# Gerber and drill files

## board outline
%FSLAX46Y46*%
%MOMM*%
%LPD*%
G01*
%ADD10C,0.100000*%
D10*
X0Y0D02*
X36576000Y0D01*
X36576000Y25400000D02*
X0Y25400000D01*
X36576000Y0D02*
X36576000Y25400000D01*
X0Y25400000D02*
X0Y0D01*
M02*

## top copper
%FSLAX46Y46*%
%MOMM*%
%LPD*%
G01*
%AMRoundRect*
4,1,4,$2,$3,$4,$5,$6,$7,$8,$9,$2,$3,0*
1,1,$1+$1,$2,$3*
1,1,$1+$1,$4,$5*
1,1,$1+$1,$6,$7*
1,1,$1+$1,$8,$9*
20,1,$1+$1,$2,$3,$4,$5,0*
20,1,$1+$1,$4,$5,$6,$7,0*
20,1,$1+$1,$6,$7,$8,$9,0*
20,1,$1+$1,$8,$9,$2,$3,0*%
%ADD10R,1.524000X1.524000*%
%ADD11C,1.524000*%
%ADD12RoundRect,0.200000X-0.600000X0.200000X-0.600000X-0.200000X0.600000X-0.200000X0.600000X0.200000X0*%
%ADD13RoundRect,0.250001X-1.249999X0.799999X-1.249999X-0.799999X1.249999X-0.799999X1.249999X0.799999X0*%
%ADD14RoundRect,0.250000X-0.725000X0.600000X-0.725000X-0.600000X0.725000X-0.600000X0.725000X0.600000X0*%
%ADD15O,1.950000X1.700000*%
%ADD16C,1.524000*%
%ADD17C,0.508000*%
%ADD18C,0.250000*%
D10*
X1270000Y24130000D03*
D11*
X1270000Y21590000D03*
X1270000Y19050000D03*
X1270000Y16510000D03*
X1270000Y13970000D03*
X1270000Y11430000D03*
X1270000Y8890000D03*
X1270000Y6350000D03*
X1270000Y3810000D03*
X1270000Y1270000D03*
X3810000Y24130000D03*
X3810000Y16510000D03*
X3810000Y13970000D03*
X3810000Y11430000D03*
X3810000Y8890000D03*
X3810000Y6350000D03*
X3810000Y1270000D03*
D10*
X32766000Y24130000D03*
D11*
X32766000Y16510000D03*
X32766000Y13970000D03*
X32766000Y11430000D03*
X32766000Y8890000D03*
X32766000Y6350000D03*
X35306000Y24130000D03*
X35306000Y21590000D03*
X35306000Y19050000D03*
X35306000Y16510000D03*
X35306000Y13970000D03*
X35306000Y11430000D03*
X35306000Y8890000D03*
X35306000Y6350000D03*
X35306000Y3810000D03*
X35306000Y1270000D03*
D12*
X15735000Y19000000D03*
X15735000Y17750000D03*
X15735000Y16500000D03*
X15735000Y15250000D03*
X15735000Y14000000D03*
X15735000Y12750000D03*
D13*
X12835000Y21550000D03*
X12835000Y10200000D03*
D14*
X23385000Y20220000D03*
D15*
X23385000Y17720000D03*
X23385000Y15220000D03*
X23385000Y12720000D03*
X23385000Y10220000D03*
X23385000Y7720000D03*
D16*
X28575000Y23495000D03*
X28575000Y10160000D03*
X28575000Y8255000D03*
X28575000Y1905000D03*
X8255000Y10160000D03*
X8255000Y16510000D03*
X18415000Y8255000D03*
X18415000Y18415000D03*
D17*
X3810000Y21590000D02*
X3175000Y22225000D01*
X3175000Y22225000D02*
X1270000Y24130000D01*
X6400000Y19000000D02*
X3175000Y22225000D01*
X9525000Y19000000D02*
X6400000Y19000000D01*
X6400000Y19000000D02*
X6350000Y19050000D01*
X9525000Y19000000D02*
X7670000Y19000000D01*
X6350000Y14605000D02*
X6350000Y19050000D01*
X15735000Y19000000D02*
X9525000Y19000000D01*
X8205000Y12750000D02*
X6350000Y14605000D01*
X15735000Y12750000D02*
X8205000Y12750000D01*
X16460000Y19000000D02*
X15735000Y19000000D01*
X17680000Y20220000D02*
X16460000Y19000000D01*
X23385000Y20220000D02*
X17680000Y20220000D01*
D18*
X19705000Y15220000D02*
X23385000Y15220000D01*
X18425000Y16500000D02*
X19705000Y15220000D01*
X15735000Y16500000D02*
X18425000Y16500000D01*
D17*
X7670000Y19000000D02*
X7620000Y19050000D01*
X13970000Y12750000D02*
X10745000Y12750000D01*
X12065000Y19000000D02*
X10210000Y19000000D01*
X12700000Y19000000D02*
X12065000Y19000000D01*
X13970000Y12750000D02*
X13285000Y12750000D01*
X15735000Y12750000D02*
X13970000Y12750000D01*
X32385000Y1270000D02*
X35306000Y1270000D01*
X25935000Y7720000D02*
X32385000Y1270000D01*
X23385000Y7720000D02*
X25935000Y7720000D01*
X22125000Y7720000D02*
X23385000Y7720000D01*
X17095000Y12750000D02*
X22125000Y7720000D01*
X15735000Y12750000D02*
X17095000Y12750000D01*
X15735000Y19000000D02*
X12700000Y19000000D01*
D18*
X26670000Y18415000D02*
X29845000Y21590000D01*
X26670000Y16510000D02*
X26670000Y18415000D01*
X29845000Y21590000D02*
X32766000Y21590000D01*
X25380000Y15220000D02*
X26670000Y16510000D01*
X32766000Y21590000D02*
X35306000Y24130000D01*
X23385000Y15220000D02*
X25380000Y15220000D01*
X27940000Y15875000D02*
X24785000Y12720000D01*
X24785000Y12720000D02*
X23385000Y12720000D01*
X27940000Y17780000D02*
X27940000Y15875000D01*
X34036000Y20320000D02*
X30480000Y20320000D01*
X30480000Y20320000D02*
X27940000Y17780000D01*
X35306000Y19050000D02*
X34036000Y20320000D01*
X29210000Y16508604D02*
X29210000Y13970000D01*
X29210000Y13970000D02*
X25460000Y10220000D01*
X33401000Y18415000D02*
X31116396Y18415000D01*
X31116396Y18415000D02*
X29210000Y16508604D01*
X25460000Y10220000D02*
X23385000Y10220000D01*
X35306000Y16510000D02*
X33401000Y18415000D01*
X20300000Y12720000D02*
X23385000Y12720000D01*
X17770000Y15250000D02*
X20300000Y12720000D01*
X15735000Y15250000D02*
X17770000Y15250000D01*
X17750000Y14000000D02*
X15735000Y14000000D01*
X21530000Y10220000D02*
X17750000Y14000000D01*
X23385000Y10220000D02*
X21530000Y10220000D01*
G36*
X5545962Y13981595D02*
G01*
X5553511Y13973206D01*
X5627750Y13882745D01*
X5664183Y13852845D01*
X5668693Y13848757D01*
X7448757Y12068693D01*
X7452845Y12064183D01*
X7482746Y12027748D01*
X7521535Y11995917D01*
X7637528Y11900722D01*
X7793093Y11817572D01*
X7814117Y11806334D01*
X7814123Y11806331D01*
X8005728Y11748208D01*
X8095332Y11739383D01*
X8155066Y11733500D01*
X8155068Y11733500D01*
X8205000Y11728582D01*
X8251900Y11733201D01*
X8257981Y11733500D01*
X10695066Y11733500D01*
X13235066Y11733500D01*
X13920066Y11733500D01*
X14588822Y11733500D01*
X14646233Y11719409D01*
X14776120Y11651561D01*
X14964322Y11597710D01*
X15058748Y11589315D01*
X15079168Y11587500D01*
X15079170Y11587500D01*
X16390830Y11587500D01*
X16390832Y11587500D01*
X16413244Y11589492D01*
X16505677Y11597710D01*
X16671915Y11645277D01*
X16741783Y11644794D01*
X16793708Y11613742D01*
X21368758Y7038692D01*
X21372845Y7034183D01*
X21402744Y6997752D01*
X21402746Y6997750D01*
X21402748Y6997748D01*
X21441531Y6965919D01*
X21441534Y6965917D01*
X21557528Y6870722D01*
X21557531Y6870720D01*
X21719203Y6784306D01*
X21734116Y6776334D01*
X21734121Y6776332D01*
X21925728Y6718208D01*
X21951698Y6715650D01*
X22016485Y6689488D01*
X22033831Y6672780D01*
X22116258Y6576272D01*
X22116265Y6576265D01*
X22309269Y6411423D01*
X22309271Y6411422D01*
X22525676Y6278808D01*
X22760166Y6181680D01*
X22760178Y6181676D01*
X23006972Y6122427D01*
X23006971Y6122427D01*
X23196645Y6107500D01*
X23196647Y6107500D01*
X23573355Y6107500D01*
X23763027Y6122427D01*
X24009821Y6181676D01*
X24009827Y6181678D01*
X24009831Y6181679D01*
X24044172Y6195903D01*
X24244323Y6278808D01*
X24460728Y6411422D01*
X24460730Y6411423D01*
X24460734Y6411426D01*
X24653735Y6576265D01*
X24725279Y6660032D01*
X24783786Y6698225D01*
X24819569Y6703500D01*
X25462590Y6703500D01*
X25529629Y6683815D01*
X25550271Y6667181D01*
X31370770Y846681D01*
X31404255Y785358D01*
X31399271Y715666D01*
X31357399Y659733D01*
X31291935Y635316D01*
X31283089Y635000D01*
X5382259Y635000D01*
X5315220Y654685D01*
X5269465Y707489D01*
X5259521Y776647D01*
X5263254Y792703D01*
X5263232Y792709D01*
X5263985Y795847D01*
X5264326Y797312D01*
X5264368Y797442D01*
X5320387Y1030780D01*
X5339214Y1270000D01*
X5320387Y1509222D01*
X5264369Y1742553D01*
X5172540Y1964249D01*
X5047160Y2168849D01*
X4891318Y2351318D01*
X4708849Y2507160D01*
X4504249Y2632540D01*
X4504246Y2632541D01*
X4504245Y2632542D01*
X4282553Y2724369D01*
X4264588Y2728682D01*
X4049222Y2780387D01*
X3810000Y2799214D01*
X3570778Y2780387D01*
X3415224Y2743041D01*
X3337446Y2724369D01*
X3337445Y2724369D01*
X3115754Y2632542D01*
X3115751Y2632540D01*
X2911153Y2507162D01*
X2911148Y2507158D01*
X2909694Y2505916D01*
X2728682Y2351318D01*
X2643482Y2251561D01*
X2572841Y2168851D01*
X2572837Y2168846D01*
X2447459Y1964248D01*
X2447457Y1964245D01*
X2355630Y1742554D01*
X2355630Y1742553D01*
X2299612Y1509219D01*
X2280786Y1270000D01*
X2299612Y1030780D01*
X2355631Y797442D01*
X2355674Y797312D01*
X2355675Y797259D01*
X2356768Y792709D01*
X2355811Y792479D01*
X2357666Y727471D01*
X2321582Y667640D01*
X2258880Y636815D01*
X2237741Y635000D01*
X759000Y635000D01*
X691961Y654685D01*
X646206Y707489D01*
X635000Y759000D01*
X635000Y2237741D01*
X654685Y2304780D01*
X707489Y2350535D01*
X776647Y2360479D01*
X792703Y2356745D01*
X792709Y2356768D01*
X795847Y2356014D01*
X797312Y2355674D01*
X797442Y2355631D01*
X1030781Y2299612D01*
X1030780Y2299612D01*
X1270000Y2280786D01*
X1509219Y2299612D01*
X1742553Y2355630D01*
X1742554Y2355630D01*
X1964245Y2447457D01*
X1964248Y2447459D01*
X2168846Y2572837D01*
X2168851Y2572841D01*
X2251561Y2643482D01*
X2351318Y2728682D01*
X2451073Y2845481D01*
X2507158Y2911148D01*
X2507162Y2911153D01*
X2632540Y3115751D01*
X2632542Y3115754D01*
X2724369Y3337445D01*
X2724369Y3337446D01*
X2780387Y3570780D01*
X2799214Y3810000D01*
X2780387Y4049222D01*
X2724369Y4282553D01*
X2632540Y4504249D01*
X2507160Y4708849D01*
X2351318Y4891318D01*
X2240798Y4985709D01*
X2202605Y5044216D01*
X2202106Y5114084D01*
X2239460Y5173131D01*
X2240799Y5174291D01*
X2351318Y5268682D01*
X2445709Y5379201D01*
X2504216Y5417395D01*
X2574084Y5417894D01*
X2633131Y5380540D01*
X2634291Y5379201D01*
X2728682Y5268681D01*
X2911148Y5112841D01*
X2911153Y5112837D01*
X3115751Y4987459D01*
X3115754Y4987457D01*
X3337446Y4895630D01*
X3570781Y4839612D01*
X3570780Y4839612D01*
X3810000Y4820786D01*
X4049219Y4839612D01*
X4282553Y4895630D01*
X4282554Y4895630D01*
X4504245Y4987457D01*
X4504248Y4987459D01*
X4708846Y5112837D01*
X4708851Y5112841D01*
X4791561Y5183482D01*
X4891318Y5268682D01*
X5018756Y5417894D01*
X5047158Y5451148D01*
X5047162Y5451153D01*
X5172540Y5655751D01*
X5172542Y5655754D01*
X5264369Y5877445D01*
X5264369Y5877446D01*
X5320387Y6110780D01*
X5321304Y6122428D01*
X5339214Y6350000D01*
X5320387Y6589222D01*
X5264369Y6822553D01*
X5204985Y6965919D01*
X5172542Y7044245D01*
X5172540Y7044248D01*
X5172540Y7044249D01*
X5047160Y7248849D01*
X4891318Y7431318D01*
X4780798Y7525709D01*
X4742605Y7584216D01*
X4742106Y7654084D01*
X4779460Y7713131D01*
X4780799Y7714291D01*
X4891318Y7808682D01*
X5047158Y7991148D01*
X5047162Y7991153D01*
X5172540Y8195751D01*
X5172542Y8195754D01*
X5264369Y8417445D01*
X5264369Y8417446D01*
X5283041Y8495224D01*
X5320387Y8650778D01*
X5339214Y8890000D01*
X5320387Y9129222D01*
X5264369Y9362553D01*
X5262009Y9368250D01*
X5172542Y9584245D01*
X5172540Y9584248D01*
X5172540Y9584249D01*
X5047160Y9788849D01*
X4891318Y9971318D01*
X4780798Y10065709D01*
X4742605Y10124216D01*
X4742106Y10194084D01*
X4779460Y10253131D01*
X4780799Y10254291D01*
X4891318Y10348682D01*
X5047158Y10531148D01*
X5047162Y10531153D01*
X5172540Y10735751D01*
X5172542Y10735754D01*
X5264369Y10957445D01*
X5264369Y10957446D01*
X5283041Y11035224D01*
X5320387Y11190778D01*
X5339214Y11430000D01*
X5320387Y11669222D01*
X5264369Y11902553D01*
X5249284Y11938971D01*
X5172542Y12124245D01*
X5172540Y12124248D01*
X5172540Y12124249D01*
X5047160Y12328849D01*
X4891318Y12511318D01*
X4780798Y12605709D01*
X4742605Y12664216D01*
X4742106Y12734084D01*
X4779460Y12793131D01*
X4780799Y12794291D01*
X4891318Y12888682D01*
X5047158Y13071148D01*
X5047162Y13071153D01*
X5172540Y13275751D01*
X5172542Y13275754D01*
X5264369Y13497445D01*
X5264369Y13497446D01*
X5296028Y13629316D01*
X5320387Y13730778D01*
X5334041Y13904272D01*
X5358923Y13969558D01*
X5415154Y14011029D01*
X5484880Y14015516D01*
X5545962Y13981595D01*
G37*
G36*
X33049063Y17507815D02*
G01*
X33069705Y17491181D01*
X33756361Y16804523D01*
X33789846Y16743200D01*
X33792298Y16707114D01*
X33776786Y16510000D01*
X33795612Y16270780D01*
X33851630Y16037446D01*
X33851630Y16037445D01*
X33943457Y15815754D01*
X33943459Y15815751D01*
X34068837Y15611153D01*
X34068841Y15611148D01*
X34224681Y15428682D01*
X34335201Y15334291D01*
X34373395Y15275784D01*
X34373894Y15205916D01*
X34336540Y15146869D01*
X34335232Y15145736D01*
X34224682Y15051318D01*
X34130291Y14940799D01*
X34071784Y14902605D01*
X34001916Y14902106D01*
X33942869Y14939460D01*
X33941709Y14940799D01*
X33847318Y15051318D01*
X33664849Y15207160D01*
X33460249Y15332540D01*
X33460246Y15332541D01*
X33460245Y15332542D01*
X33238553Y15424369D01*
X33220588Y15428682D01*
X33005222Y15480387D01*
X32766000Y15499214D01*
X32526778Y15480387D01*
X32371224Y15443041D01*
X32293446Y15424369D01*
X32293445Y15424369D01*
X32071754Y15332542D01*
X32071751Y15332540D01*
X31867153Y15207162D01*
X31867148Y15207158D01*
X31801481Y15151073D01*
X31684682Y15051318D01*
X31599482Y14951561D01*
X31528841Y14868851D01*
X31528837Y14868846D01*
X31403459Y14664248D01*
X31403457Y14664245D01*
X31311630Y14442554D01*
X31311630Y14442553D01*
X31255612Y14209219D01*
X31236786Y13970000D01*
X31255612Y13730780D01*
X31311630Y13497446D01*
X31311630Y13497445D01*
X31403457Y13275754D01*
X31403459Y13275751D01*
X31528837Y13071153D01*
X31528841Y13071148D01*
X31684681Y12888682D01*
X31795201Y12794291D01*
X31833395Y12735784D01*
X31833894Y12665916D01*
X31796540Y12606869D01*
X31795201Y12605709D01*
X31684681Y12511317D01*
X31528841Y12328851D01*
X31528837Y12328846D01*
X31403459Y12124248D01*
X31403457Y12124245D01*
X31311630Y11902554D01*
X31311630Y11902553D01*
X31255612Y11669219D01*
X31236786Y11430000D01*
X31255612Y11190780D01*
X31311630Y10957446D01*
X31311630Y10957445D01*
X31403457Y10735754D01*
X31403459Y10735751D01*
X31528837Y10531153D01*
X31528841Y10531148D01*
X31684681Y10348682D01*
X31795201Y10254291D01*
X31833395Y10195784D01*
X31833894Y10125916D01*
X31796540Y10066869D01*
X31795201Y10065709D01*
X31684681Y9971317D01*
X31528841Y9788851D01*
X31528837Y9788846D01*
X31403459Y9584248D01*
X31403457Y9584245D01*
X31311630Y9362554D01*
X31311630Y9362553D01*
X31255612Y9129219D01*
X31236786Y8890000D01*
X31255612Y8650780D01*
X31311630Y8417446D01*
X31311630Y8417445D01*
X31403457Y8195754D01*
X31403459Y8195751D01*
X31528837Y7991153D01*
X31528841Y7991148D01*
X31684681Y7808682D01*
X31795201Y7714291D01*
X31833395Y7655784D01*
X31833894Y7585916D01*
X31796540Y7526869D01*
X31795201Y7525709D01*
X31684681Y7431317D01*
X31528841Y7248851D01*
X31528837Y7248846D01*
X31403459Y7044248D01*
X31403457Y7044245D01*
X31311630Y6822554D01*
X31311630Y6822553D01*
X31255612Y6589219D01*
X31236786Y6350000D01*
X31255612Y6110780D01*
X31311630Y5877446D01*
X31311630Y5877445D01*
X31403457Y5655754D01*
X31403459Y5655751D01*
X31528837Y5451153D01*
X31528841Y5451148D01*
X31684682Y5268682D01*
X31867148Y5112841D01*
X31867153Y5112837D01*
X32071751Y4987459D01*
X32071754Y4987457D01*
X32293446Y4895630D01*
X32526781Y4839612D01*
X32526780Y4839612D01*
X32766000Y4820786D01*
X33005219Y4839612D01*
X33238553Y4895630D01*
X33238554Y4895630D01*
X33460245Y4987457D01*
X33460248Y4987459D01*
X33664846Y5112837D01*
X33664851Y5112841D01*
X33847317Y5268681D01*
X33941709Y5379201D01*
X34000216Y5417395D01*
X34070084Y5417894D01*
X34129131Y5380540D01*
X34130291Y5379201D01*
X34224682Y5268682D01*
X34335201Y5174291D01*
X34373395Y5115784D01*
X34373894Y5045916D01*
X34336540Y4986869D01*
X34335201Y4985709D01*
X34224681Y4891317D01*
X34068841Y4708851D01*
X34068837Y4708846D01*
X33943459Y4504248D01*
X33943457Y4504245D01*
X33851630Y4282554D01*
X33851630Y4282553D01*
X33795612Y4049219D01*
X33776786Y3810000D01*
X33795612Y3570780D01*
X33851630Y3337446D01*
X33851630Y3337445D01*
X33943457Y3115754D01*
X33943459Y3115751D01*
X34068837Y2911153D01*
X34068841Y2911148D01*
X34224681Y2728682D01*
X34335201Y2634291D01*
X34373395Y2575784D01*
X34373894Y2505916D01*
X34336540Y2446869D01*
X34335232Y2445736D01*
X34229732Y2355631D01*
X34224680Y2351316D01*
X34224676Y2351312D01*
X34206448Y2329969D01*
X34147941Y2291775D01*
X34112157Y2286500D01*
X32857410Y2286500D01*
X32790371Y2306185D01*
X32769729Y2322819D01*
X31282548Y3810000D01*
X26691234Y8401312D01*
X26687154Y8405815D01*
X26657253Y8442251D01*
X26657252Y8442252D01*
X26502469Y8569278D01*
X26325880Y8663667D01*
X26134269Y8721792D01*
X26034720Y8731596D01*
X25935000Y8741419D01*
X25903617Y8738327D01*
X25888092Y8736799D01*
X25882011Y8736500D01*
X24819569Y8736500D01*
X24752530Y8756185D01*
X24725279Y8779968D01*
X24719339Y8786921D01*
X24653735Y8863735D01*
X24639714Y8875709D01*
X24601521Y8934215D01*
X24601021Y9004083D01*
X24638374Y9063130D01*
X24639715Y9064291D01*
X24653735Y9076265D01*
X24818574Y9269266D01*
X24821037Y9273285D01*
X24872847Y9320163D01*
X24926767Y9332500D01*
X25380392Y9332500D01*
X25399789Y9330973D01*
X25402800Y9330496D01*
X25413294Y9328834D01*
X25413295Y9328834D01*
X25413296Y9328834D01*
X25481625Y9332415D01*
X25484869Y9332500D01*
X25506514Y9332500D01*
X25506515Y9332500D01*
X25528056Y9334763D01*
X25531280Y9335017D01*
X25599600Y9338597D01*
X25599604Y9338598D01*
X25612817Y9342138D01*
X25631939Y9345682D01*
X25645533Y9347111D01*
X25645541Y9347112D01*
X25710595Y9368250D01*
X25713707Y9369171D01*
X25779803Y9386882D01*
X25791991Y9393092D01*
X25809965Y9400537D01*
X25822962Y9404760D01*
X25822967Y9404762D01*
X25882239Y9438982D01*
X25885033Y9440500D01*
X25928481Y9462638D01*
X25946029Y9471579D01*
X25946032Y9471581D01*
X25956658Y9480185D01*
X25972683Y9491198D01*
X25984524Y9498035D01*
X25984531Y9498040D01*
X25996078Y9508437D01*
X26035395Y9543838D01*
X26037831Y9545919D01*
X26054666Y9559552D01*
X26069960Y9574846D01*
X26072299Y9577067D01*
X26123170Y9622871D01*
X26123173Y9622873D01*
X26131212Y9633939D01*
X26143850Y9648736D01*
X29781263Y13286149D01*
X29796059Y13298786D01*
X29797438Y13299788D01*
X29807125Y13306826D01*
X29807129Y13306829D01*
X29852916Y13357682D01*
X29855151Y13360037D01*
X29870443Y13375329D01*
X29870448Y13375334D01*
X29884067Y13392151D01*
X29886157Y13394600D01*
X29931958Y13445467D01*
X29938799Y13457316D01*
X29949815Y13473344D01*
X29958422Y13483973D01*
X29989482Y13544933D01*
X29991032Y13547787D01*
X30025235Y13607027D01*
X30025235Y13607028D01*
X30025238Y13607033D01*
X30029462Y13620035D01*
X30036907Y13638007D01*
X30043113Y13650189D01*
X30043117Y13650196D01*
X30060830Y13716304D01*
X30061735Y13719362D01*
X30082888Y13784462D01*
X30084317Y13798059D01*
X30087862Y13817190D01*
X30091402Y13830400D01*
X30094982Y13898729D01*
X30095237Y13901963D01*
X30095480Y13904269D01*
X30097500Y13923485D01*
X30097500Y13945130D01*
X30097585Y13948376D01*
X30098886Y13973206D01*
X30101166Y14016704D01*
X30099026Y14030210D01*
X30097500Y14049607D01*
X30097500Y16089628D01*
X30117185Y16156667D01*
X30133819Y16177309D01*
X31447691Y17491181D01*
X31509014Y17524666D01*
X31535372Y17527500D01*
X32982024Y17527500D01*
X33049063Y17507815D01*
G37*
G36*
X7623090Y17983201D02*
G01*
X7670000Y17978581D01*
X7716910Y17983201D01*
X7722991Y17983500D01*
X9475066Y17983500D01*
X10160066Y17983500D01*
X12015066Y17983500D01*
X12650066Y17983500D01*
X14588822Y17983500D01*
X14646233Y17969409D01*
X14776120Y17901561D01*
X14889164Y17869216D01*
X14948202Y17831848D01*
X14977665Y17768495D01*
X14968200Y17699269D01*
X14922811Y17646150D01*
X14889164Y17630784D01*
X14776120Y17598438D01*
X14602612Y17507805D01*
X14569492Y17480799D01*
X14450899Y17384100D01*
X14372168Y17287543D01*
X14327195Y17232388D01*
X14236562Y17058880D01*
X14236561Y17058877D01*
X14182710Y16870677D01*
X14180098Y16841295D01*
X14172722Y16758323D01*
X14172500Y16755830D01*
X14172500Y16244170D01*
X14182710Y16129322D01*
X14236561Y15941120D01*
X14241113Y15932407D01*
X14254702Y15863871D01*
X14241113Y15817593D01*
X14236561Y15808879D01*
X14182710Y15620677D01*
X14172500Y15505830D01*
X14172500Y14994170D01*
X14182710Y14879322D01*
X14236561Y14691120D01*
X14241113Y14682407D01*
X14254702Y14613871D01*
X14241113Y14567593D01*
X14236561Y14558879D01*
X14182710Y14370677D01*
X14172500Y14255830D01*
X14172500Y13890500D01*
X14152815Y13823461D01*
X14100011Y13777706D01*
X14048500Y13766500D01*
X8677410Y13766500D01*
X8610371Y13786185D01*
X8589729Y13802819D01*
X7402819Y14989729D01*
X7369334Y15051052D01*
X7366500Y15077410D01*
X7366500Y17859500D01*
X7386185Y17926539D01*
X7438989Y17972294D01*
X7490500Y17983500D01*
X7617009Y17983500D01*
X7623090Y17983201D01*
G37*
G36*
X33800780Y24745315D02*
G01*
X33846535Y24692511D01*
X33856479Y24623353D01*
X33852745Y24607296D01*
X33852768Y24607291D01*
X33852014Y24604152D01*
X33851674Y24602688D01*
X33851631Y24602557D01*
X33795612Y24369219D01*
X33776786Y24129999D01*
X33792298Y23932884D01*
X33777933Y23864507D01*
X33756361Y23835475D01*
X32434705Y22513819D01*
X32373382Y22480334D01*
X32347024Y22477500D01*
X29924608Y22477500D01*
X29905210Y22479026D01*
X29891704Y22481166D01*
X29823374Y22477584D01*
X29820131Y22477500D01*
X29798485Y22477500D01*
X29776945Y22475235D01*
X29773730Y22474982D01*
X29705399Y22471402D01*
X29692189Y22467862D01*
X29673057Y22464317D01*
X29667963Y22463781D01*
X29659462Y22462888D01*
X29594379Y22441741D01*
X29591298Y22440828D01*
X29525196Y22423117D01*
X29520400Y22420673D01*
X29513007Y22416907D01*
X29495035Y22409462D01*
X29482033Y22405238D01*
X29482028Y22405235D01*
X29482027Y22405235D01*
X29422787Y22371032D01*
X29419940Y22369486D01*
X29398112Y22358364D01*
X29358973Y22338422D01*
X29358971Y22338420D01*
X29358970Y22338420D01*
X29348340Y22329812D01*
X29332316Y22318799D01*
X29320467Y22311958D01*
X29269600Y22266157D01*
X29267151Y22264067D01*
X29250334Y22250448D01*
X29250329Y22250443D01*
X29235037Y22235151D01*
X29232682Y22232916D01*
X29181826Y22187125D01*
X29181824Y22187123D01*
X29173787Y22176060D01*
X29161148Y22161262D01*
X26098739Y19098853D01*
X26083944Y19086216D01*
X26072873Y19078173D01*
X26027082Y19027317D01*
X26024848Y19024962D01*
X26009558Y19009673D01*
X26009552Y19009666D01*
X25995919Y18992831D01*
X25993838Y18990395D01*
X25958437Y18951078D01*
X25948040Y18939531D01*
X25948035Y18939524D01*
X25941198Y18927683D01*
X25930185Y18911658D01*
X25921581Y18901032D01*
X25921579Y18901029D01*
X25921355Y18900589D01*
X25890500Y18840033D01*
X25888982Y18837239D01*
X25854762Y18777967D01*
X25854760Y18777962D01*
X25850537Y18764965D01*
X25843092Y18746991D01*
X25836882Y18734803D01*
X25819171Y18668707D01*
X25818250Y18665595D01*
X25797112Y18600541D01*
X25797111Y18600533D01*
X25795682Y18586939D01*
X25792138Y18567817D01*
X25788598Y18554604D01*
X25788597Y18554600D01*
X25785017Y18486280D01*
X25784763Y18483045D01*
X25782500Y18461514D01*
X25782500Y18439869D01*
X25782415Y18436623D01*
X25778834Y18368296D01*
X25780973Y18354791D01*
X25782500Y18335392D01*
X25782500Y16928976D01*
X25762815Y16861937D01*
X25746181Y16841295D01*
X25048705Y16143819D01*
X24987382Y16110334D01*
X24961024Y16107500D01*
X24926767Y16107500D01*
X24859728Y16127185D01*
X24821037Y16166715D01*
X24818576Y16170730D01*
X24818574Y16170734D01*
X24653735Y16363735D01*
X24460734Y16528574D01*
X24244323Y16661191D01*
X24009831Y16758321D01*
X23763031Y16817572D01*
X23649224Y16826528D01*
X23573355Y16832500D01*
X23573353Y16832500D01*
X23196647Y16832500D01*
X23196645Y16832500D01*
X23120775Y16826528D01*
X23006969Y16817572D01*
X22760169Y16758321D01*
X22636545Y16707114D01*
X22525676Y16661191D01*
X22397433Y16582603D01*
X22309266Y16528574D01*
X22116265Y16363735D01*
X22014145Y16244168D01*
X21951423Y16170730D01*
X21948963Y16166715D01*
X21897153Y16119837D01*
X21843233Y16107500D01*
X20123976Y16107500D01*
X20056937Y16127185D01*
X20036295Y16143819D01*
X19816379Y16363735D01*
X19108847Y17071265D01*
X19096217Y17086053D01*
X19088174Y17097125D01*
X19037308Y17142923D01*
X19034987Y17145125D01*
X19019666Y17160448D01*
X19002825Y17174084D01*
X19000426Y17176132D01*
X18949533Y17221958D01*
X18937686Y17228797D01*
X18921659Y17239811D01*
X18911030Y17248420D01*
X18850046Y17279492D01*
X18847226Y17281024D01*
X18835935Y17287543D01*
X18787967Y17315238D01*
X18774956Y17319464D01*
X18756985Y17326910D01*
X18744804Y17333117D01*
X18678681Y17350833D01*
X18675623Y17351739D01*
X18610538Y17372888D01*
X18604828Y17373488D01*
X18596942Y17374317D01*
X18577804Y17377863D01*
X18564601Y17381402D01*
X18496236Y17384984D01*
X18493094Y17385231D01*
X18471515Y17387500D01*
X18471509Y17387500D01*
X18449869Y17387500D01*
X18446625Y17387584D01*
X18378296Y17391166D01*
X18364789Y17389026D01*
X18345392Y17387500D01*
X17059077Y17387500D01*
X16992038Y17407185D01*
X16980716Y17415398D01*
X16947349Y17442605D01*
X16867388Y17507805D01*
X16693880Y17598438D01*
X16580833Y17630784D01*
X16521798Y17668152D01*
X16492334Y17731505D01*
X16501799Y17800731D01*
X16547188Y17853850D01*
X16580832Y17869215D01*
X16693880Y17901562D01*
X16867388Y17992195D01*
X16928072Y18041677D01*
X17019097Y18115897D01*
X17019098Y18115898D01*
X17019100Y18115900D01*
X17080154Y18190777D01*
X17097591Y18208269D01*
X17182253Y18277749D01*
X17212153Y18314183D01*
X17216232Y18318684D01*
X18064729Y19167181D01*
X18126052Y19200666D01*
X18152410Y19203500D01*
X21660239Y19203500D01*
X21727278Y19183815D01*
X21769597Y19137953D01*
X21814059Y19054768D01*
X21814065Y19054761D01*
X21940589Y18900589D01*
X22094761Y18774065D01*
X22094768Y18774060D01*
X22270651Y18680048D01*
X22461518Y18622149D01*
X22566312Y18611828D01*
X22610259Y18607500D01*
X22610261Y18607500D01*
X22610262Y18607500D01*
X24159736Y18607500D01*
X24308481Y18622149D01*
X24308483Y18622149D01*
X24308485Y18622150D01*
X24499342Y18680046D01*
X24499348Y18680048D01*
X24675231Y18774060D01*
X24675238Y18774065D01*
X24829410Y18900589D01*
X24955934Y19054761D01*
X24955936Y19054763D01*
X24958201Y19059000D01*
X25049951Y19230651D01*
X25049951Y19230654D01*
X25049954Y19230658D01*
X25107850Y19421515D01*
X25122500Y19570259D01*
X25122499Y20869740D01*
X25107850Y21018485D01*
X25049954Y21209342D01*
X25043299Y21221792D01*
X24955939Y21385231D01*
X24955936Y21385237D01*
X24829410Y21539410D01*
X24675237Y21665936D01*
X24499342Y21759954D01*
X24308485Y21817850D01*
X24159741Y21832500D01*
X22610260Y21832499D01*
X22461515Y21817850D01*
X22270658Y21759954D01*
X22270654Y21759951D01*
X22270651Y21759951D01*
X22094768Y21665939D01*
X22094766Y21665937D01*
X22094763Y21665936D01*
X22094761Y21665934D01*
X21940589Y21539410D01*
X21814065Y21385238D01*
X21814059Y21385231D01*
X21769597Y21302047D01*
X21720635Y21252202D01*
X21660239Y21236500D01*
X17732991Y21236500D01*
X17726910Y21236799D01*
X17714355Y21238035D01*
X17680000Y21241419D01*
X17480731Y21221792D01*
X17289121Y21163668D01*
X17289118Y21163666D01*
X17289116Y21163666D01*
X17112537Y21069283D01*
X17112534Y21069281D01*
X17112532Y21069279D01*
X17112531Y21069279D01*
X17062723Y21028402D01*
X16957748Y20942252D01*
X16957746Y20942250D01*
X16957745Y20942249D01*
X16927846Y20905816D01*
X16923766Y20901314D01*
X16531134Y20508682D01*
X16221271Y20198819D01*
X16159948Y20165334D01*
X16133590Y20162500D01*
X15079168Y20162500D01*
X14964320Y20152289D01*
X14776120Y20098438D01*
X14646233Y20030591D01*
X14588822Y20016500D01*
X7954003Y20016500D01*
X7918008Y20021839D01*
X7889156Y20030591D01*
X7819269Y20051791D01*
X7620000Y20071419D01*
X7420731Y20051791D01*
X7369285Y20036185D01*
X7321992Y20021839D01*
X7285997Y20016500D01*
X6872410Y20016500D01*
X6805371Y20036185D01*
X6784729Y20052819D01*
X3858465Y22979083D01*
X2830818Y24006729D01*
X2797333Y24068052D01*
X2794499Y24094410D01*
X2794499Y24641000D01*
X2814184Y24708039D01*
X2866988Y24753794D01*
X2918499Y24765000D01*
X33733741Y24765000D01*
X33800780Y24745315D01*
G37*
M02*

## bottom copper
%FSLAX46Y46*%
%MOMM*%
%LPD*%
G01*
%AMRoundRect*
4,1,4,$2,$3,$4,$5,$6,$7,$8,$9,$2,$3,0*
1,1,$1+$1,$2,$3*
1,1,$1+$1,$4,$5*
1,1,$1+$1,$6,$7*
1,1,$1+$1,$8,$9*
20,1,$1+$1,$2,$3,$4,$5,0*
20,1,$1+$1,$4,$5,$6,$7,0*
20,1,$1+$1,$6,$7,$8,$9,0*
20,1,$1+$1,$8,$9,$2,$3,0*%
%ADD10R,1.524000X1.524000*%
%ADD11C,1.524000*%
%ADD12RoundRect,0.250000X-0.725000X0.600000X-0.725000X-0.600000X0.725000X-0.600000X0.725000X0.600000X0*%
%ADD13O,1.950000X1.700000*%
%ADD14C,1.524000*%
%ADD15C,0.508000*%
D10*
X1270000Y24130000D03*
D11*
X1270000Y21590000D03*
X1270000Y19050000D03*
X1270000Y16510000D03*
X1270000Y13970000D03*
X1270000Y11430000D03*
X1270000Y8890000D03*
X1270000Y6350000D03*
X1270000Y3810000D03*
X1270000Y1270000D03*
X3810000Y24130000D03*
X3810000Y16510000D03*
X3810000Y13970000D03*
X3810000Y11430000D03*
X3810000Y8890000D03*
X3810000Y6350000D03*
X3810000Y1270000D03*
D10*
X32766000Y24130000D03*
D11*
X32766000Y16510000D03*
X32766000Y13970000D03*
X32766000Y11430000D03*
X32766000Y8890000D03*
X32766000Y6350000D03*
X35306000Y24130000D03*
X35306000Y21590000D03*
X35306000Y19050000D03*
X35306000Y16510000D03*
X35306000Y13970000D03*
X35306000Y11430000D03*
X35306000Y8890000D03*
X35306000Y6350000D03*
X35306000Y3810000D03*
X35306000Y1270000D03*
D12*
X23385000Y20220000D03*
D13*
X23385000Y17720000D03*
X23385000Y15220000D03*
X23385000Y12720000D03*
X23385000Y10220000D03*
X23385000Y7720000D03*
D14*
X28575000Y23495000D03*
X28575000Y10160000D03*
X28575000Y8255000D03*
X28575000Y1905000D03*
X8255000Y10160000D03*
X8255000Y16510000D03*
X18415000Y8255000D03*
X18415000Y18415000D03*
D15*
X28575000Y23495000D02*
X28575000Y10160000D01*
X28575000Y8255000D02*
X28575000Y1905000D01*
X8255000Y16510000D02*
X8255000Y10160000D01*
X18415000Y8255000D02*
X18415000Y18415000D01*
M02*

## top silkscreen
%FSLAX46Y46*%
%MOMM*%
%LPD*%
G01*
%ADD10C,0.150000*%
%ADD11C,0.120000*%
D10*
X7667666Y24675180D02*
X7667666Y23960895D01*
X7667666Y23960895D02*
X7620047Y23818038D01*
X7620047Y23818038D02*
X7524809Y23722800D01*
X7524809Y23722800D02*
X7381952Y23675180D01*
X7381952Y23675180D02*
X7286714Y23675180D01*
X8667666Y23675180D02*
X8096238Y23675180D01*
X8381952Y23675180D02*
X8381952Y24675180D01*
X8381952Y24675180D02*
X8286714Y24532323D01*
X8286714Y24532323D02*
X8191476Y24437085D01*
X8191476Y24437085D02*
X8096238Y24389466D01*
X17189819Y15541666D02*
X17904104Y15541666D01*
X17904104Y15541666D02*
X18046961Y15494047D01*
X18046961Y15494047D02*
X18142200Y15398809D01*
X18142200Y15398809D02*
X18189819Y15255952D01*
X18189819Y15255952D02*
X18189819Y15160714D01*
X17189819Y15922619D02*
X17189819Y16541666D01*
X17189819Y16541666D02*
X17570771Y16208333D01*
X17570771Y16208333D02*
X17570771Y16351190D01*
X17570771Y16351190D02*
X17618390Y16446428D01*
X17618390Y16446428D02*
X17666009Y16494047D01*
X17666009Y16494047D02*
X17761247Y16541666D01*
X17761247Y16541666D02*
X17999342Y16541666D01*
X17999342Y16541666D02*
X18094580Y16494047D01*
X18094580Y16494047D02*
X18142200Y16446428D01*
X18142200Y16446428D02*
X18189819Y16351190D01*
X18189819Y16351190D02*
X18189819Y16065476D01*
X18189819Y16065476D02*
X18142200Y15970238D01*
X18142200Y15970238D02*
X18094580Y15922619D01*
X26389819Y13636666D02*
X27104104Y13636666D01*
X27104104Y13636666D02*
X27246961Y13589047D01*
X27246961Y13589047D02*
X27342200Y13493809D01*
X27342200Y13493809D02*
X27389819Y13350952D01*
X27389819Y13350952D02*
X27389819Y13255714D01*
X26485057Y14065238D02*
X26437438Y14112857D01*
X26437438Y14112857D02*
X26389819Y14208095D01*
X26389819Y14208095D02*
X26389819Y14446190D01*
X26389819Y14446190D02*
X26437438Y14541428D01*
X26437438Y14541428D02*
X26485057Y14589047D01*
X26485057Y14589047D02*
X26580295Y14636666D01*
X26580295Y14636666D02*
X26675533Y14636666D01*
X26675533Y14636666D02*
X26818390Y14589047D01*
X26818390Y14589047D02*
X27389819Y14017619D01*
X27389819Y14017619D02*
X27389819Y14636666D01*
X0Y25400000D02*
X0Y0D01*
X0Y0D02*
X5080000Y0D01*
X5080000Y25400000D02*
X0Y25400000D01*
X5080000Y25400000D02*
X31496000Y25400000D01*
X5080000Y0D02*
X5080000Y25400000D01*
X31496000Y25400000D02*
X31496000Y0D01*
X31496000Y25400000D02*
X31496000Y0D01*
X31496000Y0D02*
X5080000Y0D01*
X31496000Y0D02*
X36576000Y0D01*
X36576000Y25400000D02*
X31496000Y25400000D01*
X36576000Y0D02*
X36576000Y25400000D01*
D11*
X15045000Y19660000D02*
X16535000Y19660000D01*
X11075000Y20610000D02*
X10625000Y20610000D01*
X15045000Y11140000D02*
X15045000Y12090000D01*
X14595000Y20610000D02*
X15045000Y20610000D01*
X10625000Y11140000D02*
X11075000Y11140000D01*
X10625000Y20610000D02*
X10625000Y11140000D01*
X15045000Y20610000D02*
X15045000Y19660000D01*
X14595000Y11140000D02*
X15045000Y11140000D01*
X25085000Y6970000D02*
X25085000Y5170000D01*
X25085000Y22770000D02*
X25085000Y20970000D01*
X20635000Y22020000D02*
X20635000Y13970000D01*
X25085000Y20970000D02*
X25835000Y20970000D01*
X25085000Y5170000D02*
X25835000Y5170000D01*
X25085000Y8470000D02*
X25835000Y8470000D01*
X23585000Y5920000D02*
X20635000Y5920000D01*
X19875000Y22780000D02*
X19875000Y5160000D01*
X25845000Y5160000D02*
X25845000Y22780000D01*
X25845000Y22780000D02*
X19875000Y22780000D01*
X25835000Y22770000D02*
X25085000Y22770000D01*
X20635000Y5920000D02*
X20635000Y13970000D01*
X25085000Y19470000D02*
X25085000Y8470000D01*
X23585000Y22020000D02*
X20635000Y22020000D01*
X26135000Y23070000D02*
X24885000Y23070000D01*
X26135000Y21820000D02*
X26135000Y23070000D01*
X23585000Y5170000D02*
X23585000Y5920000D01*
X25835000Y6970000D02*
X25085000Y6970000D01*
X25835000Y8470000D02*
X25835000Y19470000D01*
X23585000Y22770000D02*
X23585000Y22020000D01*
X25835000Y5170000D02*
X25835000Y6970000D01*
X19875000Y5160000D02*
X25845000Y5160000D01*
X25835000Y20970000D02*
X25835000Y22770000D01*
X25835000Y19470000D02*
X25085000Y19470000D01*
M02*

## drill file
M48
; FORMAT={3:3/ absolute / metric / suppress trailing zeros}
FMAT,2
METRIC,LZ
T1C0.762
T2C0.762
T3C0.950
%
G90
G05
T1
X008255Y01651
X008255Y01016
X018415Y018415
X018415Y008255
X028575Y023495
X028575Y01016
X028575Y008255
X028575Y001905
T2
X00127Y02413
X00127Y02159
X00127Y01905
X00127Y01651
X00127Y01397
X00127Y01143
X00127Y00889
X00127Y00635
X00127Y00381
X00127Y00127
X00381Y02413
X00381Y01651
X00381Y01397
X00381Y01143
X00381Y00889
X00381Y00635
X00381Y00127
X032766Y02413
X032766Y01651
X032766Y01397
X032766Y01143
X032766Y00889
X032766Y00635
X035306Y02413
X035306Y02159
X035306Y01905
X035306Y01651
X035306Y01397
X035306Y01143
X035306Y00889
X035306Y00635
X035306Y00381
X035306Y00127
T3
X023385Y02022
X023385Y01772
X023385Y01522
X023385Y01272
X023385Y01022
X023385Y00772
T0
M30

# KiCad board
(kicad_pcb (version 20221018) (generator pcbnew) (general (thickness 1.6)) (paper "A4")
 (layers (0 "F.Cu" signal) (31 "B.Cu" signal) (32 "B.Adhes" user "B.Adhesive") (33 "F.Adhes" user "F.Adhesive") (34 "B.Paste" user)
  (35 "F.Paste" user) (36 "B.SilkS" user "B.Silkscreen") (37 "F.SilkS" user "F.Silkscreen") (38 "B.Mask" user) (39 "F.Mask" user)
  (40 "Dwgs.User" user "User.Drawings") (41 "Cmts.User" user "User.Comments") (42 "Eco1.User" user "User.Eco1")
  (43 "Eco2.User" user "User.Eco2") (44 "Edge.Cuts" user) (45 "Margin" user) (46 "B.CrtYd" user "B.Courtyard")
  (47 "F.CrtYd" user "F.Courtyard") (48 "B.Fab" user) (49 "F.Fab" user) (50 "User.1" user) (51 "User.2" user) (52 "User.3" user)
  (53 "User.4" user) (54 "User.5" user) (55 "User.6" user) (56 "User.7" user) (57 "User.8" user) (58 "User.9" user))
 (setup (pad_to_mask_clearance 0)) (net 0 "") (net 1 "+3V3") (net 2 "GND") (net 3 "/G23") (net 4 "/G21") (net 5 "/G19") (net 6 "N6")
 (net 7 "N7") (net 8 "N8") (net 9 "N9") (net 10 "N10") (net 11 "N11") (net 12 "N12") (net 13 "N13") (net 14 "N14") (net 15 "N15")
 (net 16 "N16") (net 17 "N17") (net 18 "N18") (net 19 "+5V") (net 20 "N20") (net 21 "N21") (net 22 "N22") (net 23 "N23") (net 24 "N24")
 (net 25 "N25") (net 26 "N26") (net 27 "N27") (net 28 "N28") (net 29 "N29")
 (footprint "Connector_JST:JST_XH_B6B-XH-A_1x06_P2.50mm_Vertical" (layer "F.Cu") (at 23.385 -20.22 -90)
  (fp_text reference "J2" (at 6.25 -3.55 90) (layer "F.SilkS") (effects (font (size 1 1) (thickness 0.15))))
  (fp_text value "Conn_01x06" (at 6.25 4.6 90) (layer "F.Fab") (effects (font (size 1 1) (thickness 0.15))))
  (fp_line (start -2.85 -2.75) (end -2.85 -1.5) (stroke (width 0.12) (type solid)) (layer "F.SilkS"))
  (fp_line (start -2.56 -2.46) (end -2.56 3.51) (stroke (width 0.12) (type solid)) (layer "F.SilkS"))
  (fp_line (start -2.56 3.51) (end 15.06 3.51) (stroke (width 0.12) (type solid)) (layer "F.SilkS"))
  (fp_line (start -2.55 -2.45) (end -2.55 -1.7) (stroke (width 0.12) (type solid)) (layer "F.SilkS"))
  (fp_line (start -2.55 -1.7) (end -0.75 -1.7) (stroke (width 0.12) (type solid)) (layer "F.SilkS"))
  (fp_line (start -2.55 -0.2) (end -1.8 -0.2) (stroke (width 0.12) (type solid)) (layer "F.SilkS"))
  (fp_line (start -1.8 -0.2) (end -1.8 2.75) (stroke (width 0.12) (type solid)) (layer "F.SilkS"))
  (fp_line (start -1.8 2.75) (end 6.25 2.75) (stroke (width 0.12) (type solid)) (layer "F.SilkS"))
  (fp_line (start -1.6 -2.75) (end -2.85 -2.75) (stroke (width 0.12) (type solid)) (layer "F.SilkS"))
  (fp_line (start -0.75 -2.45) (end -2.55 -2.45) (stroke (width 0.12) (type solid)) (layer "F.SilkS"))
  (fp_line (start -0.75 -1.7) (end -0.75 -2.45) (stroke (width 0.12) (type solid)) (layer "F.SilkS"))
  (fp_line (start 0.75 -2.45) (end 0.75 -1.7) (stroke (width 0.12) (type solid)) (layer "F.SilkS"))
  (fp_line (start 0.75 -1.7) (end 11.75 -1.7) (stroke (width 0.12) (type solid)) (layer "F.SilkS"))
  (fp_line (start 11.75 -2.45) (end 0.75 -2.45) (stroke (width 0.12) (type solid)) (layer "F.SilkS"))
  (fp_line (start 11.75 -1.7) (end 11.75 -2.45) (stroke (width 0.12) (type solid)) (layer "F.SilkS"))
  (fp_line (start 13.25 -2.45) (end 13.25 -1.7) (stroke (width 0.12) (type solid)) (layer "F.SilkS"))
  (fp_line (start 13.25 -1.7) (end 15.05 -1.7) (stroke (width 0.12) (type solid)) (layer "F.SilkS"))
  (fp_line (start 14.3 -0.2) (end 14.3 2.75) (stroke (width 0.12) (type solid)) (layer "F.SilkS"))
  (fp_line (start 14.3 2.75) (end 6.25 2.75) (stroke (width 0.12) (type solid)) (layer "F.SilkS"))
  (fp_line (start 15.05 -2.45) (end 13.25 -2.45) (stroke (width 0.12) (type solid)) (layer "F.SilkS"))
  (fp_line (start 15.05 -1.7) (end 15.05 -2.45) (stroke (width 0.12) (type solid)) (layer "F.SilkS"))
  (fp_line (start 15.05 -0.2) (end 14.3 -0.2) (stroke (width 0.12) (type solid)) (layer "F.SilkS"))
  (fp_line (start 15.06 -2.46) (end -2.56 -2.46) (stroke (width 0.12) (type solid)) (layer "F.SilkS"))
  (fp_line (start 15.06 3.51) (end 15.06 -2.46) (stroke (width 0.12) (type solid)) (layer "F.SilkS"))
  (pad "1" thru_hole roundrect (at 0 0 270) (size 1.7 1.95) (drill 0.95) (layers "*.Cu" "*.Mask") (roundrect_rratio 0.1470588235)
   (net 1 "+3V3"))
  (pad "2" thru_hole oval (at 2.5 0 270) (size 1.7 1.95) (drill 0.95) (layers "*.Cu" "*.Mask") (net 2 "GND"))
  (pad "3" thru_hole oval (at 5 0 270) (size 1.7 1.95) (drill 0.95) (layers "*.Cu" "*.Mask") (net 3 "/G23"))
  (pad "4" thru_hole oval (at 7.5 0 270) (size 1.7 1.95) (drill 0.95) (layers "*.Cu" "*.Mask") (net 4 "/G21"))
  (pad "5" thru_hole oval (at 10 0 270) (size 1.7 1.95) (drill 0.95) (layers "*.Cu" "*.Mask") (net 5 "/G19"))
  (pad "6" thru_hole oval (at 12.5 0 270) (size 1.7 1.95) (drill 0.95) (layers "*.Cu" "*.Mask") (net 1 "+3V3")))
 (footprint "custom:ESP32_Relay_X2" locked (layer "F.Cu") (at 35.306 -13.97)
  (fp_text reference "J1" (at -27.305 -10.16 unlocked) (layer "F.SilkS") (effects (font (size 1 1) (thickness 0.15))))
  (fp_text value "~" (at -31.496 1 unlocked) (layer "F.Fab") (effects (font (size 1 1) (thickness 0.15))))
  (fp_line (start -35.306 -11.43) (end -35.306 13.97) (stroke (width 0.15) (type default)) (layer "F.SilkS"))
  (fp_line (start -35.306 13.97) (end -30.226 13.97) (stroke (width 0.15) (type default)) (layer "F.SilkS"))
  (fp_line (start -30.226 -11.43) (end -35.306 -11.43) (stroke (width 0.15) (type default)) (layer "F.SilkS"))
  (fp_line (start -30.226 -11.43) (end -3.81 -11.43) (stroke (width 0.15) (type default)) (layer "F.SilkS"))
  (fp_line (start -30.226 13.97) (end -30.226 -11.43) (stroke (width 0.15) (type default)) (layer "F.SilkS"))
  (fp_line (start -3.81 -11.43) (end -3.81 13.97) (stroke (width 0.15) (type default)) (layer "F.SilkS"))
  (fp_line (start -3.81 -11.43) (end -3.81 13.97) (stroke (width 0.15) (type default)) (layer "F.SilkS"))
  (fp_line (start -3.81 13.97) (end -30.226 13.97) (stroke (width 0.15) (type default)) (layer "F.SilkS"))
  (fp_line (start -3.81 13.97) (end 1.27 13.97) (stroke (width 0.15) (type default)) (layer "F.SilkS"))
  (fp_line (start 1.27 -11.43) (end -3.81 -11.43) (stroke (width 0.15) (type default)) (layer "F.SilkS"))
  (fp_line (start 1.27 13.97) (end 1.27 -11.43) (stroke (width 0.15) (type default)) (layer "F.SilkS"))
  (pad "1" thru_hole rect locked (at -34.036 -10.16) (size 1.524 1.524) (drill 0.762) (layers "*.Cu" "*.Mask") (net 1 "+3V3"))
  (pad "2" thru_hole circle locked (at -34.036 -7.62) (size 1.524 1.524) (drill 0.762) (layers "*.Cu" "*.Mask") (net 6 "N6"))
  (pad "3" thru_hole circle locked (at -34.036 -5.08) (size 1.524 1.524) (drill 0.762) (layers "*.Cu" "*.Mask") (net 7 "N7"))
  (pad "4" thru_hole circle locked (at -34.036 -2.54) (size 1.524 1.524) (drill 0.762) (layers "*.Cu" "*.Mask") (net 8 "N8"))
  (pad "5" thru_hole circle locked (at -34.036 0) (size 1.524 1.524) (drill 0.762) (layers "*.Cu" "*.Mask") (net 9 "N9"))
  (pad "6" thru_hole circle locked (at -34.036 2.54) (size 1.524 1.524) (drill 0.762) (layers "*.Cu" "*.Mask") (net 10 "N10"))
  (pad "7" thru_hole circle locked (at -34.036 5.08) (size 1.524 1.524) (drill 0.762) (layers "*.Cu" "*.Mask") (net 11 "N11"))
  (pad "8" thru_hole circle locked (at -34.036 7.62) (size 1.524 1.524) (drill 0.762) (layers "*.Cu" "*.Mask") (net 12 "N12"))
  (pad "9" thru_hole circle locked (at -34.036 10.16) (size 1.524 1.524) (drill 0.762) (layers "*.Cu" "*.Mask") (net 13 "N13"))
  (pad "10" thru_hole circle locked (at -34.036 12.7) (size 1.524 1.524) (drill 0.762) (layers "*.Cu" "*.Mask") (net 2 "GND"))
  (pad "11" thru_hole circle locked (at -31.496 -10.16) (size 1.524 1.524) (drill 0.762) (layers "*.Cu" "*.Mask") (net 2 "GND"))
  (pad "14" thru_hole circle locked (at -31.496 -2.54) (size 1.524 1.524) (drill 0.762) (layers "*.Cu" "*.Mask") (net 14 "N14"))
  (pad "15" thru_hole circle locked (at -31.496 0) (size 1.524 1.524) (drill 0.762) (layers "*.Cu" "*.Mask") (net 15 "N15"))
  (pad "16" thru_hole circle locked (at -31.496 2.54) (size 1.524 1.524) (drill 0.762) (layers "*.Cu" "*.Mask") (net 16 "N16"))
  (pad "17" thru_hole circle locked (at -31.496 5.08) (size 1.524 1.524) (drill 0.762) (layers "*.Cu" "*.Mask") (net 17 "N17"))
  (pad "18" thru_hole circle locked (at -31.496 7.62) (size 1.524 1.524) (drill 0.762) (layers "*.Cu" "*.Mask") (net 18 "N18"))
  (pad "20" thru_hole circle locked (at -31.496 12.7) (size 1.524 1.524) (drill 0.762) (layers "*.Cu" "*.Mask") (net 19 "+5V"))
  (pad "21" thru_hole rect locked (at -2.54 -10.16) (size 1.524 1.524) (drill 0.762) (layers "*.Cu" "*.Mask") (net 2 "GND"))
  (pad "24" thru_hole circle locked (at -2.54 -2.54) (size 1.524 1.524) (drill 0.762) (layers "*.Cu" "*.Mask") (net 2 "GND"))
  (pad "25" thru_hole circle locked (at -2.54 0) (size 1.524 1.524) (drill 0.762) (layers "*.Cu" "*.Mask") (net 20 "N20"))
  (pad "26" thru_hole circle locked (at -2.54 2.54) (size 1.524 1.524) (drill 0.762) (layers "*.Cu" "*.Mask") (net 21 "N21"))
  (pad "27" thru_hole circle locked (at -2.54 5.08) (size 1.524 1.524) (drill 0.762) (layers "*.Cu" "*.Mask") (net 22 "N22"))
  (pad "28" thru_hole circle locked (at -2.54 7.62) (size 1.524 1.524) (drill 0.762) (layers "*.Cu" "*.Mask") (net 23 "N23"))
  (pad "31" thru_hole circle locked (at 0 -10.16) (size 1.524 1.524) (drill 0.762) (layers "*.Cu" "*.Mask") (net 3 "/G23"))
  (pad "32" thru_hole circle locked (at 0 -7.62) (size 1.524 1.524) (drill 0.762) (layers "*.Cu" "*.Mask") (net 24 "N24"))
  (pad "33" thru_hole circle locked (at 0 -5.08) (size 1.524 1.524) (drill 0.762) (layers "*.Cu" "*.Mask") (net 4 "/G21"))
  (pad "34" thru_hole circle locked (at 0 -2.54) (size 1.524 1.524) (drill 0.762) (layers "*.Cu" "*.Mask") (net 5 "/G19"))
  (pad "35" thru_hole circle locked (at 0 0) (size 1.524 1.524) (drill 0.762) (layers "*.Cu" "*.Mask") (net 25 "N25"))
  (pad "36" thru_hole circle locked (at 0 2.54) (size 1.524 1.524) (drill 0.762) (layers "*.Cu" "*.Mask") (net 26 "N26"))
  (pad "37" thru_hole circle locked (at 0 5.08) (size 1.524 1.524) (drill 0.762) (layers "*.Cu" "*.Mask") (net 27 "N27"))
  (pad "38" thru_hole circle locked (at 0 7.62) (size 1.524 1.524) (drill 0.762) (layers "*.Cu" "*.Mask") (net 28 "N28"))
  (pad "39" thru_hole circle locked (at 0 10.16) (size 1.524 1.524) (drill 0.762) (layers "*.Cu" "*.Mask") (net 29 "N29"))
  (pad "40" thru_hole circle locked (at 0 12.7) (size 1.524 1.524) (drill 0.762) (layers "*.Cu" "*.Mask") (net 1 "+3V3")))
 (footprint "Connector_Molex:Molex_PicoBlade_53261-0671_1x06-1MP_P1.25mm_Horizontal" (layer "F.Cu") (at 13.335 -15.875 -90)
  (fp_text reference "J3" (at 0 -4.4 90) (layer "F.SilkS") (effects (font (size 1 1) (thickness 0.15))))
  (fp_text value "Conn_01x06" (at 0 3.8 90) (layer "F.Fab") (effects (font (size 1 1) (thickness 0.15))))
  (fp_line (start -4.735 -1.71) (end -3.785 -1.71) (stroke (width 0.12) (type solid)) (layer "F.SilkS"))
  (fp_line (start -4.735 -1.26) (end -4.735 -1.71) (stroke (width 0.12) (type solid)) (layer "F.SilkS"))
  (fp_line (start -4.735 2.26) (end -4.735 2.71) (stroke (width 0.12) (type solid)) (layer "F.SilkS"))
  (fp_line (start -4.735 2.71) (end 4.735 2.71) (stroke (width 0.12) (type solid)) (layer "F.SilkS"))
  (fp_line (start -3.785 -1.71) (end -3.785 -3.2) (stroke (width 0.12) (type solid)) (layer "F.SilkS"))
  (fp_line (start 4.735 -1.71) (end 3.785 -1.71) (stroke (width 0.12) (type solid)) (layer "F.SilkS"))
  (fp_line (start 4.735 -1.26) (end 4.735 -1.71) (stroke (width 0.12) (type solid)) (layer "F.SilkS"))
  (fp_line (start 4.735 2.71) (end 4.735 2.26) (stroke (width 0.12) (type solid)) (layer "F.SilkS"))
  (pad "1" smd roundrect (at -3.125 -2.4 270) (size 0.8 1.6) (layers "F.Cu" "F.Paste" "F.Mask") (roundrect_rratio 0.25) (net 1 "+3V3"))
  (pad "2" smd roundrect (at -1.875 -2.4 270) (size 0.8 1.6) (layers "F.Cu" "F.Paste" "F.Mask") (roundrect_rratio 0.25) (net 2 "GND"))
  (pad "3" smd roundrect (at -0.625 -2.4 270) (size 0.8 1.6) (layers "F.Cu" "F.Paste" "F.Mask") (roundrect_rratio 0.25) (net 3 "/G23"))
  (pad "4" smd roundrect (at 0.625 -2.4 270) (size 0.8 1.6) (layers "F.Cu" "F.Paste" "F.Mask") (roundrect_rratio 0.25) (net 4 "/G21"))
  (pad "5" smd roundrect (at 1.875 -2.4 270) (size 0.8 1.6) (layers "F.Cu" "F.Paste" "F.Mask") (roundrect_rratio 0.25) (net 5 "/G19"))
  (pad "6" smd roundrect (at 3.125 -2.4 270) (size 0.8 1.6) (layers "F.Cu" "F.Paste" "F.Mask") (roundrect_rratio 0.25) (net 1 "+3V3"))
  (pad "MP" smd roundrect (at -5.675 0.5 270) (size 2.1 3) (layers "F.Cu" "F.Paste" "F.Mask") (roundrect_rratio 0.1190480952))
  (pad "MP" smd roundrect (at 5.675 0.5 270) (size 2.1 3) (layers "F.Cu" "F.Paste" "F.Mask") (roundrect_rratio 0.1190480952)))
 (gr_line (start 0 0) (end 36.576 0) (stroke (width 0.1) (type default)) (layer "Edge.Cuts"))
 (gr_line (start 36.576 -25.4) (end 0 -25.4) (stroke (width 0.1) (type default)) (layer "Edge.Cuts"))
 (gr_line (start 36.576 0) (end 36.576 -25.4) (stroke (width 0.1) (type default)) (layer "Edge.Cuts"))
 (gr_line (start 0 -25.4) (end 0 0) (stroke (width 0.1) (type default)) (layer "Edge.Cuts"))
 (segment (start 3.175 -22.225) (end 1.27 -24.13) (width 0.508) (layer "F.Cu") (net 1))
 (segment (start 25.935 -7.72) (end 32.385 -1.27) (width 0.508) (layer "F.Cu") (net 1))
 (segment (start 9.525 -19) (end 6.4 -19) (width 0.508) (layer "F.Cu") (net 1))
 (segment (start 6.4 -19) (end 3.175 -22.225) (width 0.508) (layer "F.Cu") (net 1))
 (segment (start 9.525 -19) (end 7.67 -19) (width 0.508) (layer "F.Cu") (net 1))
 (segment (start 23.385 -7.72) (end 25.935 -7.72) (width 0.508) (layer "F.Cu") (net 1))
 (segment (start 12.7 -19) (end 12.065 -19) (width 0.508) (layer "F.Cu") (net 1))
 (segment (start 13.97 -12.75) (end 13.285 -12.75) (width 0.508) (layer "F.Cu") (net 1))
 (segment (start 22.125 -7.72) (end 23.385 -7.72) (width 0.508) (layer "F.Cu") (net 1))
 (segment (start 15.735 -19) (end 12.7 -19) (width 0.508) (layer "F.Cu") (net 1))
 (segment (start 23.385 -20.22) (end 17.68 -20.22) (width 0.508) (layer "F.Cu") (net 1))
 (segment (start 16.46 -19) (end 15.735 -19) (width 0.508) (layer "F.Cu") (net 1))
 (segment (start 15.735 -12.75) (end 13.97 -12.75) (width 0.508) (layer "F.Cu") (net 1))
 (segment (start 3.81 -21.59) (end 3.175 -22.225) (width 0.508) (layer "F.Cu") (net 1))
 (segment (start 7.67 -19) (end 7.62 -19.05) (width 0.508) (layer "F.Cu") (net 1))
 (segment (start 15.735 -12.75) (end 17.095 -12.75) (width 0.508) (layer "F.Cu") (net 1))
 (segment (start 13.97 -12.75) (end 10.745 -12.75) (width 0.508) (layer "F.Cu") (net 1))
 (segment (start 6.35 -14.605) (end 6.35 -19.05) (width 0.508) (layer "F.Cu") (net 1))
 (segment (start 17.095 -12.75) (end 22.125 -7.72) (width 0.508) (layer "F.Cu") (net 1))
 (segment (start 17.68 -20.22) (end 16.46 -19) (width 0.508) (layer "F.Cu") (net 1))
 (segment (start 15.735 -12.75) (end 8.205 -12.75) (width 0.508) (layer "F.Cu") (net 1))
 (segment (start 32.385 -1.27) (end 35.306 -1.27) (width 0.508) (layer "F.Cu") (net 1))
 (segment (start 15.735 -19) (end 9.525 -19) (width 0.508) (layer "F.Cu") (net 1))
 (segment (start 8.205 -12.75) (end 6.35 -14.605) (width 0.508) (layer "F.Cu") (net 1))
 (segment (start 6.4 -19) (end 6.35 -19.05) (width 0.508) (layer "F.Cu") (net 1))
 (segment (start 12.065 -19) (end 10.21 -19) (width 0.508) (layer "F.Cu") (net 1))
 (via (at 8.255 -10.16) (size 1.524) (drill 0.762) (layers "F.Cu" "B.Cu") (free) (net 2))
 (via (at 8.255 -16.51) (size 1.524) (drill 0.762) (layers "F.Cu" "B.Cu") (free) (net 2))
 (via (at 28.575 -10.16) (size 1.524) (drill 0.762) (layers "F.Cu" "B.Cu") (free) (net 2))
 (via (at 28.575 -1.905) (size 1.524) (drill 0.762) (layers "F.Cu" "B.Cu") (free) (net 2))
 (via (at 28.575 -8.255) (size 1.524) (drill 0.762) (layers "F.Cu" "B.Cu") (free) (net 2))
 (via (at 18.415 -8.255) (size 1.524) (drill 0.762) (layers "F.Cu" "B.Cu") (free) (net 2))
 (via (at 28.575 -23.495) (size 1.524) (drill 0.762) (layers "F.Cu" "B.Cu") (free) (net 2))
 (via (at 18.415 -18.415) (size 1.524) (drill 0.762) (layers "F.Cu" "B.Cu") (free) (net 2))
 (segment (start 28.575 -23.495) (end 28.575 -10.16) (width 0.508) (layer "B.Cu") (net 2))
 (segment (start 28.575 -8.255) (end 28.575 -1.905) (width 0.508) (layer "B.Cu") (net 2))
 (segment (start 18.415 -8.255) (end 18.415 -18.415) (width 0.508) (layer "B.Cu") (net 2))
 (segment (start 8.255 -16.51) (end 8.255 -10.16) (width 0.508) (layer "B.Cu") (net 2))
 (segment (start 32.766 -21.59) (end 35.306 -24.13) (width 0.25) (layer "F.Cu") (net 3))
 (segment (start 19.705 -15.22) (end 23.385 -15.22) (width 0.25) (layer "F.Cu") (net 3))
 (segment (start 29.845 -21.59) (end 32.766 -21.59) (width 0.25) (layer "F.Cu") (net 3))
 (segment (start 23.385 -15.22) (end 25.38 -15.22) (width 0.25) (layer "F.Cu") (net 3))
 (segment (start 26.67 -16.51) (end 26.67 -18.415) (width 0.25) (layer "F.Cu") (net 3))
 (segment (start 25.38 -15.22) (end 26.67 -16.51) (width 0.25) (layer "F.Cu") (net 3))
 (segment (start 15.735 -16.5) (end 18.425 -16.5) (width 0.25) (layer "F.Cu") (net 3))
 (segment (start 18.425 -16.5) (end 19.705 -15.22) (width 0.25) (layer "F.Cu") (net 3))
 (segment (start 26.67 -18.415) (end 29.845 -21.59) (width 0.25) (layer "F.Cu") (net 3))
 (segment (start 34.036 -20.32) (end 30.48 -20.32) (width 0.25) (layer "F.Cu") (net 4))
 (segment (start 30.48 -20.32) (end 27.94 -17.78) (width 0.25) (layer "F.Cu") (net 4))
 (segment (start 17.77 -15.25) (end 20.3 -12.72) (width 0.25) (layer "F.Cu") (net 4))
 (segment (start 35.306 -19.05) (end 34.036 -20.32) (width 0.25) (layer "F.Cu") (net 4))
 (segment (start 24.785 -12.72) (end 23.385 -12.72) (width 0.25) (layer "F.Cu") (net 4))
 (segment (start 15.735 -15.25) (end 17.77 -15.25) (width 0.25) (layer "F.Cu") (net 4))
 (segment (start 27.94 -17.78) (end 27.94 -15.875) (width 0.25) (layer "F.Cu") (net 4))
 (segment (start 27.94 -15.875) (end 24.785 -12.72) (width 0.25) (layer "F.Cu") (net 4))
 (segment (start 20.3 -12.72) (end 23.385 -12.72) (width 0.25) (layer "F.Cu") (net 4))
 (segment (start 25.46 -10.22) (end 23.385 -10.22) (width 0.25) (layer "F.Cu") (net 5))
 (segment (start 21.53 -10.22) (end 17.75 -14) (width 0.25) (layer "F.Cu") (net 5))
 (segment (start 29.21 -16.508604) (end 29.21 -13.97) (width 0.25) (layer "F.Cu") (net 5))
 (segment (start 17.75 -14) (end 15.735 -14) (width 0.25) (layer "F.Cu") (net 5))
 (segment (start 33.401 -18.415) (end 31.116396 -18.415) (width 0.25) (layer "F.Cu") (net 5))
 (segment (start 35.306 -16.51) (end 33.401 -18.415) (width 0.25) (layer "F.Cu") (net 5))
 (segment (start 29.21 -13.97) (end 25.46 -10.22) (width 0.25) (layer "F.Cu") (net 5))
 (segment (start 31.116396 -18.415) (end 29.21 -16.508604) (width 0.25) (layer "F.Cu") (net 5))
 (segment (start 23.385 -10.22) (end 21.53 -10.22) (width 0.25) (layer "F.Cu") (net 5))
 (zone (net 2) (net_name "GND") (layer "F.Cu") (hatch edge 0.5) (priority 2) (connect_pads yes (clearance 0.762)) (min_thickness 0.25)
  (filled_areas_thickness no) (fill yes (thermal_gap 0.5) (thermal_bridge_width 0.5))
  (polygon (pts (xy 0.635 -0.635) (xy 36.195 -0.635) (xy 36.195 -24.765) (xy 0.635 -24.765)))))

